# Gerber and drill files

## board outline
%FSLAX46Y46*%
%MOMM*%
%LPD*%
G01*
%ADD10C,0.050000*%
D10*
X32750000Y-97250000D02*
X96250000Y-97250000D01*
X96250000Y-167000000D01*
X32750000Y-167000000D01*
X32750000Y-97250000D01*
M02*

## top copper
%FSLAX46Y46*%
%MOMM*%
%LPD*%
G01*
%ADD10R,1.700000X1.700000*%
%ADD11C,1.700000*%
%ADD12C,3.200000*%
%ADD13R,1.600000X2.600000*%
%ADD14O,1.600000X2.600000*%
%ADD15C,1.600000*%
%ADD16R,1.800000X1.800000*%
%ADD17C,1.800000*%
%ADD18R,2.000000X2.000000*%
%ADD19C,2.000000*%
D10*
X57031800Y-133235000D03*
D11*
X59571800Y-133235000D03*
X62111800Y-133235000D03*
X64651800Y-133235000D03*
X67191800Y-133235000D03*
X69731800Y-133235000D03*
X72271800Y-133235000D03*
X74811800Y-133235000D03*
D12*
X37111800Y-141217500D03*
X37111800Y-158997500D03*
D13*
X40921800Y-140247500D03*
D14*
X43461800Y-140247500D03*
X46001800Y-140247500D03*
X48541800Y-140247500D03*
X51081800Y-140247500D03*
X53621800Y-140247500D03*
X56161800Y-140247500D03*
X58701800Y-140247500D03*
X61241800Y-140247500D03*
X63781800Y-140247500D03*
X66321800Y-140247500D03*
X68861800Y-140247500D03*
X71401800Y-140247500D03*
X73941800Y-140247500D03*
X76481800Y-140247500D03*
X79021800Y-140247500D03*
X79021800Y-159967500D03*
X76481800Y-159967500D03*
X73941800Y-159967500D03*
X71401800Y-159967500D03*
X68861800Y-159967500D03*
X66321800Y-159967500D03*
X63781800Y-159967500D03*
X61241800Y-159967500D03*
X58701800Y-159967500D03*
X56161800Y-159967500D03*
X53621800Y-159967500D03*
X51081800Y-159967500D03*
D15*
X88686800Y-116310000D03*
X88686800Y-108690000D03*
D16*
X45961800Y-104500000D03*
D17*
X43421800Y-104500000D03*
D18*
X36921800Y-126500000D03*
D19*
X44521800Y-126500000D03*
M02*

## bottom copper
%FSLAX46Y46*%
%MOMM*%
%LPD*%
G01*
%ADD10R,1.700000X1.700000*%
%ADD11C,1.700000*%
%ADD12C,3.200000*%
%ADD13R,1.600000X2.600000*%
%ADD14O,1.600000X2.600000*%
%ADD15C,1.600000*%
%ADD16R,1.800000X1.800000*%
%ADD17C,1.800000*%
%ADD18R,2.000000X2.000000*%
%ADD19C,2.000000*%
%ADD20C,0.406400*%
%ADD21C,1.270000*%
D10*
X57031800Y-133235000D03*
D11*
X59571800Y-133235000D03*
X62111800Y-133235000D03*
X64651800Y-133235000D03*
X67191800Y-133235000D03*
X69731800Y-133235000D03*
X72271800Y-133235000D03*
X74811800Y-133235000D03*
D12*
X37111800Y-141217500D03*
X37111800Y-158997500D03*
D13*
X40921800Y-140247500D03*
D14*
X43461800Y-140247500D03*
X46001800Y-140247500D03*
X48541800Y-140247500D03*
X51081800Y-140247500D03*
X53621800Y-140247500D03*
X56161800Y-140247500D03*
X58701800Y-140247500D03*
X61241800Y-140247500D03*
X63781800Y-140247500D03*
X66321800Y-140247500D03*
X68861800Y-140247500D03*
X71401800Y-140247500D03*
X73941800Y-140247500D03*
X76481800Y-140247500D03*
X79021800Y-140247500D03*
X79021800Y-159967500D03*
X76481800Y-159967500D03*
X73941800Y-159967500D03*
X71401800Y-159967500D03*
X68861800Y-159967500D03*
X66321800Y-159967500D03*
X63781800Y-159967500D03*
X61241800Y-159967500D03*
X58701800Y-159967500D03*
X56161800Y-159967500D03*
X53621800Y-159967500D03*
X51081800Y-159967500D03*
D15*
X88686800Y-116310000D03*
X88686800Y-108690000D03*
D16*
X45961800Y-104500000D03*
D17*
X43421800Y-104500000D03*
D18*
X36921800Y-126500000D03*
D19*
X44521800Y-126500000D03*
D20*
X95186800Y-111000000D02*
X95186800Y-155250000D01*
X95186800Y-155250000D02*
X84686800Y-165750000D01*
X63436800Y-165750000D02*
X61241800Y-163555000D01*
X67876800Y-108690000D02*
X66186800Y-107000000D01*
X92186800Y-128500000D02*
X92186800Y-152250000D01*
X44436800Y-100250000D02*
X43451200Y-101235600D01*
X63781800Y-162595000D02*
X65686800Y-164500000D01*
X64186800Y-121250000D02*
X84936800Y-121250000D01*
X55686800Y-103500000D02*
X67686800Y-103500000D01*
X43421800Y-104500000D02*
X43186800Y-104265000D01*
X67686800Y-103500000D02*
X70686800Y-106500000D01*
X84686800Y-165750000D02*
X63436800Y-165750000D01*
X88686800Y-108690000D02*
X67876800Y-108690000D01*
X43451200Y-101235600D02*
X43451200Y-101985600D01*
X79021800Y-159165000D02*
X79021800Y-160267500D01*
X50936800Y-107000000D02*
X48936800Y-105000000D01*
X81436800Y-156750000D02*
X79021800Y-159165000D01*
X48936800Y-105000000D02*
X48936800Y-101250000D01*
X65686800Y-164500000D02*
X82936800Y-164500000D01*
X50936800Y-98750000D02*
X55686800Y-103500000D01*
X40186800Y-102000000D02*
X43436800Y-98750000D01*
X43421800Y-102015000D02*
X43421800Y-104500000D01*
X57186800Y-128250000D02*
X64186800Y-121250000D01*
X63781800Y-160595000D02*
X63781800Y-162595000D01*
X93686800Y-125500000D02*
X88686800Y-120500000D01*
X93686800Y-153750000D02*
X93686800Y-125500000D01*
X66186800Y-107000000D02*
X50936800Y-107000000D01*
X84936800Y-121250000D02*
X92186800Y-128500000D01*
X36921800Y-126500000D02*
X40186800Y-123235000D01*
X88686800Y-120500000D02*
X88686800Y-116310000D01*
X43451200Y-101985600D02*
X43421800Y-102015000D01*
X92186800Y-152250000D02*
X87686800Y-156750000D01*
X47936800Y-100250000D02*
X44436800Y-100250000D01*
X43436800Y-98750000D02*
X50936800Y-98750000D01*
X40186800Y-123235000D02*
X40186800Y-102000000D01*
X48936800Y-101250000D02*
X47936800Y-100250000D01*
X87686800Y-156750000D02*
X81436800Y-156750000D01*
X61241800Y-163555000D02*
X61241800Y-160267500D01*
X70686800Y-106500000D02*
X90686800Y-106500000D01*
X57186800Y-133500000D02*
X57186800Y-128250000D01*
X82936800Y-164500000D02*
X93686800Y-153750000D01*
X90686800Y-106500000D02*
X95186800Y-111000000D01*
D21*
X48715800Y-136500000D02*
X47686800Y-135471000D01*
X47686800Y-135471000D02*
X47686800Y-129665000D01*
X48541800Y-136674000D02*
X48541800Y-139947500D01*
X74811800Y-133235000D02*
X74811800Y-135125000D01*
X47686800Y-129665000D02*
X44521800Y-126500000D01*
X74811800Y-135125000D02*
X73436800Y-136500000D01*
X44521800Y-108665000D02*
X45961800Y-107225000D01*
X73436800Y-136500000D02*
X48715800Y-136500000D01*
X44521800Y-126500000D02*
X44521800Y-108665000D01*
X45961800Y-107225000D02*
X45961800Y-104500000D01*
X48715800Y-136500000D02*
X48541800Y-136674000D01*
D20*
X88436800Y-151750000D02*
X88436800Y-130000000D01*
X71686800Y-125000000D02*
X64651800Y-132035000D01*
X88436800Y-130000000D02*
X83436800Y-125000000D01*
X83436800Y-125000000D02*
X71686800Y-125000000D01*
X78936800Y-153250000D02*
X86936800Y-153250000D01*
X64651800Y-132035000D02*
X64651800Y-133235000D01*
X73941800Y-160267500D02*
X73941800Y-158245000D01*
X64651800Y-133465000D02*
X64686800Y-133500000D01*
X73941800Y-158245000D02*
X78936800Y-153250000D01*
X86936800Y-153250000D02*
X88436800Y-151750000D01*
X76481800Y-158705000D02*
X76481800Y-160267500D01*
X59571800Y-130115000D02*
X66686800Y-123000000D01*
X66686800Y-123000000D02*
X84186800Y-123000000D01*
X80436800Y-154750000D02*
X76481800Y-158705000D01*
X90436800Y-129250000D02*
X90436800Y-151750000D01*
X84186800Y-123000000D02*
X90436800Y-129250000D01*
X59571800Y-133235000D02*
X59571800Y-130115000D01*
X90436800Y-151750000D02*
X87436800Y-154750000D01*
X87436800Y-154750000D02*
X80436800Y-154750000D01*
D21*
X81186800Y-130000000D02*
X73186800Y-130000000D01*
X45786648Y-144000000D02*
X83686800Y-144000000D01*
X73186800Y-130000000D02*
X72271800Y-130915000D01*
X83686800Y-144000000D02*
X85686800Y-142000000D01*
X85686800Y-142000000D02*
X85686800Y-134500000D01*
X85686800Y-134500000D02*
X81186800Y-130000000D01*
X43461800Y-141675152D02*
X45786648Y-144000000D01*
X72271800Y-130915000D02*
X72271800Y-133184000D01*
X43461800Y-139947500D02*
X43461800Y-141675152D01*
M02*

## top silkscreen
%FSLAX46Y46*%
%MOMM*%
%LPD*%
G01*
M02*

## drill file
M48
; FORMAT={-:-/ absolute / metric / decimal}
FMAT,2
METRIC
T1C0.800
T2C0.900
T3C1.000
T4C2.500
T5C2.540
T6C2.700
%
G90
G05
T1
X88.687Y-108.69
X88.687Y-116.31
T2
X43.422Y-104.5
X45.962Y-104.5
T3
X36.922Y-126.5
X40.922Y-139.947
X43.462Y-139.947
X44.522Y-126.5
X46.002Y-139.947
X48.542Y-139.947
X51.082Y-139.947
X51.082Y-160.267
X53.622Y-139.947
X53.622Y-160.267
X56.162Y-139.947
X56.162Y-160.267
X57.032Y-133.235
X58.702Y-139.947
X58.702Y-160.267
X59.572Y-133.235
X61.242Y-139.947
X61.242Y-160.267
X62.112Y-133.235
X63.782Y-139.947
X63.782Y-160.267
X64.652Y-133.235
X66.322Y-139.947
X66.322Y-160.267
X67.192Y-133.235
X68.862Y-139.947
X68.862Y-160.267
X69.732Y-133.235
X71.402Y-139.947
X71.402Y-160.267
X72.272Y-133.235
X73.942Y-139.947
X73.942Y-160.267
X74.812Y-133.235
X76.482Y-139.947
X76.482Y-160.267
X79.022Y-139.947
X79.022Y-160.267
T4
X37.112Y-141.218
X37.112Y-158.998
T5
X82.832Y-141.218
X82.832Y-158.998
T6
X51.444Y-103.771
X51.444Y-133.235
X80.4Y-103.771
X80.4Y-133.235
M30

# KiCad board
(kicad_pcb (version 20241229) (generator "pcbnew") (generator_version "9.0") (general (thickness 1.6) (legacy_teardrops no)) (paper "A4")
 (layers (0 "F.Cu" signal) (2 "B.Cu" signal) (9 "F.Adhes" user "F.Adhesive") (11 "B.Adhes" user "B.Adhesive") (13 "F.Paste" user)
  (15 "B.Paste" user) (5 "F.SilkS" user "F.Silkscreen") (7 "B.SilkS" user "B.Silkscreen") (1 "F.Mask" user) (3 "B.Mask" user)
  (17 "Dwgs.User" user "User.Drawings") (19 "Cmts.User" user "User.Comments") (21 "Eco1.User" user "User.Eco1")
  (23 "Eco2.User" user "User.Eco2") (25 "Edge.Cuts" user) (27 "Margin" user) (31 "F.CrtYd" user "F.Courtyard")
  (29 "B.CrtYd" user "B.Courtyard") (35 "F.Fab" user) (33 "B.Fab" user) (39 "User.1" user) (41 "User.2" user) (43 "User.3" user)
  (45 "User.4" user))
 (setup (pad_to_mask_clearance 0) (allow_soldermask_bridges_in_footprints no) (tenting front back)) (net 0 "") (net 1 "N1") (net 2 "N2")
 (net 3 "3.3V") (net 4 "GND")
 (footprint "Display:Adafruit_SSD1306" (layer "B.Cu") (at 57.0318 133.235)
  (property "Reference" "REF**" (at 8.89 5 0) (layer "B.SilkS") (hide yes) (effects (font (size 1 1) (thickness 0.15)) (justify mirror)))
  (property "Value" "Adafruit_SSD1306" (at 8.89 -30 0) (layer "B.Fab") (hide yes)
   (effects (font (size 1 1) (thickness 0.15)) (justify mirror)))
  (pad "" np_thru_hole circle (at -5.588 -29.464) (size 2.7 2.7) (drill 2.7) (layers "*.Cu" "*.Mask"))
  (pad "" np_thru_hole circle (at -5.588 0) (size 2.7 2.7) (drill 2.7) (layers "*.Cu" "*.Mask"))
  (pad "" np_thru_hole circle (at 23.368 -29.464) (size 2.7 2.7) (drill 2.7) (layers "*.Cu" "*.Mask"))
  (pad "" np_thru_hole circle (at 23.368 0) (size 2.7 2.7) (drill 2.7) (layers "*.Cu" "*.Mask"))
  (pad "1" thru_hole rect (at 0 0) (size 1.7 1.7) (drill 1) (layers "*.Cu" "*.Mask") (remove_unused_layers no))
  (pad "2" thru_hole circle (at 2.54 0) (size 1.7 1.7) (drill 1) (layers "*.Cu" "*.Mask") (remove_unused_layers no) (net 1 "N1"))
  (pad "3" thru_hole circle (at 5.08 0) (size 1.7 1.7) (drill 1) (layers "*.Cu" "*.Mask") (remove_unused_layers no))
  (pad "4" thru_hole circle (at 7.62 0) (size 1.7 1.7) (drill 1) (layers "*.Cu" "*.Mask") (remove_unused_layers no) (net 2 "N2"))
  (pad "5" thru_hole circle (at 10.16 0) (size 1.7 1.7) (drill 1) (layers "*.Cu" "*.Mask") (remove_unused_layers no))
  (pad "6" thru_hole circle (at 12.7 0) (size 1.7 1.7) (drill 1) (layers "*.Cu" "*.Mask") (remove_unused_layers no))
  (pad "7" thru_hole circle (at 15.24 0) (size 1.7 1.7) (drill 1) (layers "*.Cu" "*.Mask") (remove_unused_layers no) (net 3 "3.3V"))
  (pad "8" thru_hole circle (at 17.78 0) (size 1.7 1.7) (drill 1) (layers "*.Cu" "*.Mask") (remove_unused_layers no) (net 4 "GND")))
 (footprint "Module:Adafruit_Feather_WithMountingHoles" (layer "B.Cu") (at 40.9218 139.9475 -90)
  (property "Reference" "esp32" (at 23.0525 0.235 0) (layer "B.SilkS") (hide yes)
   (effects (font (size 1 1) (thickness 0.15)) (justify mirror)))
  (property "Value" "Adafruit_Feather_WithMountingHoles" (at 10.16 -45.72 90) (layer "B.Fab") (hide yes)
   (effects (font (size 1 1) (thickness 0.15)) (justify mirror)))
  (pad "" np_thru_hole circle (at 1.27 -41.91) (size 2.54 2.54) (drill 2.54) (layers "*.Cu" "*.Mask"))
  (pad "" np_thru_hole circle (at 1.27 3.81) (size 3.2 3.2) (drill 2.5) (layers "*.Cu" "*.Mask"))
  (pad "" np_thru_hole circle (at 19.05 -41.91) (size 2.54 2.54) (drill 2.54) (layers "*.Cu" "*.Mask"))
  (pad "" np_thru_hole circle (at 19.05 3.81) (size 3.2 3.2) (drill 2.5) (layers "*.Cu" "*.Mask"))
  (pad "1" thru_hole rect (at 0 0 270) (size 2.6 1.6) (drill 1 (offset 0.3 0)) (layers "*.Cu" "*.Mask") (remove_unused_layers no))
  (pad "2" thru_hole oval (at 0 -2.54 270) (size 2.6 1.6) (drill 1 (offset 0.3 0)) (layers "*.Cu" "*.Mask") (remove_unused_layers no)
   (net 3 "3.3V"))
  (pad "3" thru_hole oval (at 0 -5.08 270) (size 2.6 1.6) (drill 1 (offset 0.3 0)) (layers "*.Cu" "*.Mask") (remove_unused_layers no))
  (pad "4" thru_hole oval (at 0 -7.62 270) (size 2.6 1.6) (drill 1 (offset 0.3 0)) (layers "*.Cu" "*.Mask") (remove_unused_layers no)
   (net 4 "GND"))
  (pad "5" thru_hole oval (at 0 -10.16 270) (size 2.6 1.6) (drill 1 (offset 0.3 0)) (layers "*.Cu" "*.Mask") (remove_unused_layers no))
  (pad "6" thru_hole oval (at 0 -12.7 270) (size 2.6 1.6) (drill 1 (offset 0.3 0)) (layers "*.Cu" "*.Mask") (remove_unused_layers no))
  (pad "7" thru_hole oval (at 0 -15.24 270) (size 2.6 1.6) (drill 1 (offset 0.3 0)) (layers "*.Cu" "*.Mask") (remove_unused_layers no))
  (pad "8" thru_hole oval (at 0 -17.78 270) (size 2.6 1.6) (drill 1 (offset 0.3 0)) (layers "*.Cu" "*.Mask") (remove_unused_layers no))
  (pad "9" thru_hole oval (at 0 -20.32 270) (size 2.6 1.6) (drill 1 (offset 0.3 0)) (layers "*.Cu" "*.Mask") (remove_unused_layers no))
  (pad "10" thru_hole oval (at 0 -22.86 270) (size 2.6 1.6) (drill 1 (offset 0.3 0)) (layers "*.Cu" "*.Mask") (remove_unused_layers no))
  (pad "11" thru_hole oval (at 0 -25.4 270) (size 2.6 1.6) (drill 1 (offset 0.3 0)) (layers "*.Cu" "*.Mask") (remove_unused_layers no))
  (pad "12" thru_hole oval (at 0 -27.94 270) (size 2.6 1.6) (drill 1 (offset 0.3 0)) (layers "*.Cu" "*.Mask") (remove_unused_layers no))
  (pad "13" thru_hole oval (at 0 -30.48 270) (size 2.6 1.6) (drill 1 (offset 0.3 0)) (layers "*.Cu" "*.Mask") (remove_unused_layers no))
  (pad "14" thru_hole oval (at 0 -33.02 270) (size 2.6 1.6) (drill 1 (offset 0.3 0)) (layers "*.Cu" "*.Mask") (remove_unused_layers no))
  (pad "15" thru_hole oval (at 0 -35.56 270) (size 2.6 1.6) (drill 1 (offset 0.3 0)) (layers "*.Cu" "*.Mask") (remove_unused_layers no))
  (pad "16" thru_hole oval (at 0 -38.1 270) (size 2.6 1.6) (drill 1 (offset 0.3 0)) (layers "*.Cu" "*.Mask") (remove_unused_layers no))
  (pad "17" thru_hole oval (at 20.32 -38.1 90) (size 2.6 1.6) (drill 1 (offset 0.3 0)) (layers "*.Cu" "*.Mask") (remove_unused_layers no))
  (pad "18" thru_hole oval (at 20.32 -35.56 90) (size 2.6 1.6) (drill 1 (offset 0.3 0)) (layers "*.Cu" "*.Mask") (remove_unused_layers no)
   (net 1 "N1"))
  (pad "19" thru_hole oval (at 20.32 -33.02 90) (size 2.6 1.6) (drill 1 (offset 0.3 0)) (layers "*.Cu" "*.Mask") (remove_unused_layers no)
   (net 2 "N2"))
  (pad "20" thru_hole oval (at 20.32 -30.48 90) (size 2.6 1.6) (drill 1 (offset 0.3 0)) (layers "*.Cu" "*.Mask") (remove_unused_layers no))
  (pad "21" thru_hole oval (at 20.32 -27.94 90) (size 2.6 1.6) (drill 1 (offset 0.3 0)) (layers "*.Cu" "*.Mask") (remove_unused_layers no))
  (pad "22" thru_hole oval (at 20.32 -25.4 90) (size 2.6 1.6) (drill 1 (offset 0.3 0)) (layers "*.Cu" "*.Mask") (remove_unused_layers no))
  (pad "23" thru_hole oval (at 20.32 -22.86 90) (size 2.6 1.6) (drill 1 (offset 0.3 0)) (layers "*.Cu" "*.Mask") (remove_unused_layers no))
  (pad "24" thru_hole oval (at 20.32 -20.32 90) (size 2.6 1.6) (drill 1 (offset 0.3 0)) (layers "*.Cu" "*.Mask") (remove_unused_layers no))
  (pad "25" thru_hole oval (at 20.32 -17.78 90) (size 2.6 1.6) (drill 1 (offset 0.3 0)) (layers "*.Cu" "*.Mask") (remove_unused_layers no))
  (pad "26" thru_hole oval (at 20.32 -15.24 90) (size 2.6 1.6) (drill 1 (offset 0.3 0)) (layers "*.Cu" "*.Mask") (remove_unused_layers no))
  (pad "27" thru_hole oval (at 20.32 -12.7 90) (size 2.6 1.6) (drill 1 (offset 0.3 0)) (layers "*.Cu" "*.Mask") (remove_unused_layers no))
  (pad "28" thru_hole oval (at 20.32 -10.16 90) (size 2.6 1.6) (drill 1 (offset 0.3 0)) (layers "*.Cu" "*.Mask") (remove_unused_layers no)))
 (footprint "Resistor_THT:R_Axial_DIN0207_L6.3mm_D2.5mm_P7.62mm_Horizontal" (layer "B.Cu") (at 88.6868 116.31 90)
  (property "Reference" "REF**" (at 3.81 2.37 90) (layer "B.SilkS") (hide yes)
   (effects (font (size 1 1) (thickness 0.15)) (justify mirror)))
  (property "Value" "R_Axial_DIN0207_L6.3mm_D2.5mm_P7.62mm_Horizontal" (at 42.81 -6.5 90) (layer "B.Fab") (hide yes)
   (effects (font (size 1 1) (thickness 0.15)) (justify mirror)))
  (pad "1" thru_hole circle (at 0 0 90) (size 1.6 1.6) (drill 0.8) (layers "*.Cu" "*.Mask") (remove_unused_layers no))
  (pad "2" thru_hole circle (at 7.62 0 90) (size 1.6 1.6) (drill 0.8) (layers "*.Cu" "*.Mask") (remove_unused_layers no)))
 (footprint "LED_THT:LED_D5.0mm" (layer "B.Cu") (at 45.9618 104.5 180)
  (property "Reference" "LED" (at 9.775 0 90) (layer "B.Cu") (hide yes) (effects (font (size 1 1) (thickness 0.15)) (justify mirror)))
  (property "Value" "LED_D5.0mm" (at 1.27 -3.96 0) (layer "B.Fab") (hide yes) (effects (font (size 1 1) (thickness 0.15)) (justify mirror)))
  (pad "1" thru_hole rect (at 0 0 180) (size 1.8 1.8) (drill 0.9) (layers "*.Cu" "*.Mask") (remove_unused_layers no) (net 4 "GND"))
  (pad "2" thru_hole circle (at 2.54 0 180) (size 1.8 1.8) (drill 0.9) (layers "*.Cu" "*.Mask") (remove_unused_layers no)))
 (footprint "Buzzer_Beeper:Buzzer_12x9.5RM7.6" (layer "B.Cu") (at 36.9218 126.5)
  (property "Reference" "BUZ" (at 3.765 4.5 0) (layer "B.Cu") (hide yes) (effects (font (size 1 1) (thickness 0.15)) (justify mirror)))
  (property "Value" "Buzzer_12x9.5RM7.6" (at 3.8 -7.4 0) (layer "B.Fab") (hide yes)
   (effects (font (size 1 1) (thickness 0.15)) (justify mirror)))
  (pad "1" thru_hole rect (at 0 0) (size 2 2) (drill 1) (layers "*.Cu" "*.Mask") (remove_unused_layers no))
  (pad "2" thru_hole circle (at 7.6 0) (size 2 2) (drill 1) (layers "*.Cu" "*.Mask") (remove_unused_layers no) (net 4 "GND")))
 (gr_rect (start 32.75 97.25) (end 96.25 167) (stroke (width 0.05) (type default)) (fill no) (layer "Edge.Cuts"))
 (segment (start 95.1868 111) (end 95.1868 155.25) (width 0.4064) (layer "B.Cu") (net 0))
 (segment (start 95.1868 155.25) (end 84.6868 165.75) (width 0.4064) (layer "B.Cu") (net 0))
 (segment (start 63.4368 165.75) (end 61.2418 163.555) (width 0.4064) (layer "B.Cu") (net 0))
 (segment (start 67.8768 108.69) (end 66.1868 107) (width 0.4064) (layer "B.Cu") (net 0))
 (segment (start 92.1868 128.5) (end 92.1868 152.25) (width 0.4064) (layer "B.Cu") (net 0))
 (segment (start 44.4368 100.25) (end 43.4512 101.2356) (width 0.4064) (layer "B.Cu") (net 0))
 (segment (start 63.7818 162.595) (end 65.6868 164.5) (width 0.4064) (layer "B.Cu") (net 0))
 (segment (start 64.1868 121.25) (end 84.9368 121.25) (width 0.4064) (layer "B.Cu") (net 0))
 (segment (start 55.6868 103.5) (end 67.6868 103.5) (width 0.4064) (layer "B.Cu") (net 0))
 (segment (start 43.4218 104.5) (end 43.1868 104.265) (width 0.4064) (layer "B.Cu") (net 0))
 (segment (start 67.6868 103.5) (end 70.6868 106.5) (width 0.4064) (layer "B.Cu") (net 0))
 (segment (start 84.6868 165.75) (end 63.4368 165.75) (width 0.4064) (layer "B.Cu") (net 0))
 (segment (start 88.6868 108.69) (end 67.8768 108.69) (width 0.4064) (layer "B.Cu") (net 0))
 (segment (start 43.4512 101.2356) (end 43.4512 101.9856) (width 0.4064) (layer "B.Cu") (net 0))
 (segment (start 79.0218 159.165) (end 79.0218 160.2675) (width 0.4064) (layer "B.Cu") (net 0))
 (segment (start 50.9368 107) (end 48.9368 105) (width 0.4064) (layer "B.Cu") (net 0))
 (segment (start 81.4368 156.75) (end 79.0218 159.165) (width 0.4064) (layer "B.Cu") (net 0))
 (segment (start 48.9368 105) (end 48.9368 101.25) (width 0.4064) (layer "B.Cu") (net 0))
 (segment (start 65.6868 164.5) (end 82.9368 164.5) (width 0.4064) (layer "B.Cu") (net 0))
 (segment (start 50.9368 98.75) (end 55.6868 103.5) (width 0.4064) (layer "B.Cu") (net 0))
 (segment (start 40.1868 102) (end 43.4368 98.75) (width 0.4064) (layer "B.Cu") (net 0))
 (segment (start 43.4218 102.015) (end 43.4218 104.5) (width 0.4064) (layer "B.Cu") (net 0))
 (segment (start 57.1868 128.25) (end 64.1868 121.25) (width 0.4064) (layer "B.Cu") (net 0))
 (segment (start 63.7818 160.595) (end 63.7818 162.595) (width 0.4064) (layer "B.Cu") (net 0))
 (segment (start 93.6868 125.5) (end 88.6868 120.5) (width 0.4064) (layer "B.Cu") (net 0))
 (segment (start 93.6868 153.75) (end 93.6868 125.5) (width 0.4064) (layer "B.Cu") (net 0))
 (segment (start 66.1868 107) (end 50.9368 107) (width 0.4064) (layer "B.Cu") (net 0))
 (segment (start 84.9368 121.25) (end 92.1868 128.5) (width 0.4064) (layer "B.Cu") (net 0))
 (segment (start 36.9218 126.5) (end 40.1868 123.235) (width 0.4064) (layer "B.Cu") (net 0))
 (segment (start 88.6868 120.5) (end 88.6868 116.31) (width 0.4064) (layer "B.Cu") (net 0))
 (segment (start 43.4512 101.9856) (end 43.4218 102.015) (width 0.4064) (layer "B.Cu") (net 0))
 (segment (start 92.1868 152.25) (end 87.6868 156.75) (width 0.4064) (layer "B.Cu") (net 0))
 (segment (start 47.9368 100.25) (end 44.4368 100.25) (width 0.4064) (layer "B.Cu") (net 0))
 (segment (start 43.4368 98.75) (end 50.9368 98.75) (width 0.4064) (layer "B.Cu") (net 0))
 (segment (start 40.1868 123.235) (end 40.1868 102) (width 0.4064) (layer "B.Cu") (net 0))
 (segment (start 48.9368 101.25) (end 47.9368 100.25) (width 0.4064) (layer "B.Cu") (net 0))
 (segment (start 87.6868 156.75) (end 81.4368 156.75) (width 0.4064) (layer "B.Cu") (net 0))
 (segment (start 61.2418 163.555) (end 61.2418 160.2675) (width 0.4064) (layer "B.Cu") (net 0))
 (segment (start 70.6868 106.5) (end 90.6868 106.5) (width 0.4064) (layer "B.Cu") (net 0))
 (segment (start 57.1868 133.5) (end 57.1868 128.25) (width 0.4064) (layer "B.Cu") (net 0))
 (segment (start 82.9368 164.5) (end 93.6868 153.75) (width 0.4064) (layer "B.Cu") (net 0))
 (segment (start 90.6868 106.5) (end 95.1868 111) (width 0.4064) (layer "B.Cu") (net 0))
 (segment (start 48.7158 136.5) (end 47.6868 135.471) (width 1.27) (layer "B.Cu") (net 4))
 (segment (start 47.6868 135.471) (end 47.6868 129.665) (width 1.27) (layer "B.Cu") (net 4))
 (segment (start 48.5418 136.674) (end 48.5418 139.9475) (width 1.27) (layer "B.Cu") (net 4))
 (segment (start 74.8118 133.235) (end 74.8118 135.125) (width 1.27) (layer "B.Cu") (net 4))
 (segment (start 47.6868 129.665) (end 44.5218 126.5) (width 1.27) (layer "B.Cu") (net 4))
 (segment (start 74.8118 135.125) (end 73.4368 136.5) (width 1.27) (layer "B.Cu") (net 4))
 (segment (start 44.5218 108.665) (end 45.9618 107.225) (width 1.27) (layer "B.Cu") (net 4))
 (segment (start 73.4368 136.5) (end 48.7158 136.5) (width 1.27) (layer "B.Cu") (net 4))
 (segment (start 44.5218 126.5) (end 44.5218 108.665) (width 1.27) (layer "B.Cu") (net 4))
 (segment (start 45.9618 107.225) (end 45.9618 104.5) (width 1.27) (layer "B.Cu") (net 4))
 (segment (start 48.7158 136.5) (end 48.5418 136.674) (width 1.27) (layer "B.Cu") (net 4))
 (segment (start 88.4368 151.75) (end 88.4368 130) (width 0.4064) (layer "B.Cu") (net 2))
 (segment (start 71.6868 125) (end 64.6518 132.035) (width 0.4064) (layer "B.Cu") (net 2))
 (segment (start 88.4368 130) (end 83.4368 125) (width 0.4064) (layer "B.Cu") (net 2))
 (segment (start 83.4368 125) (end 71.6868 125) (width 0.4064) (layer "B.Cu") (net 2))
 (segment (start 78.9368 153.25) (end 86.9368 153.25) (width 0.4064) (layer "B.Cu") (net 2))
 (segment (start 64.6518 132.035) (end 64.6518 133.235) (width 0.4064) (layer "B.Cu") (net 2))
 (segment (start 73.9418 160.2675) (end 73.9418 158.245) (width 0.4064) (layer "B.Cu") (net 2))
 (segment (start 64.6518 133.465) (end 64.6868 133.5) (width 0.4064) (layer "B.Cu") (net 2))
 (segment (start 73.9418 158.245) (end 78.9368 153.25) (width 0.4064) (layer "B.Cu") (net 2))
 (segment (start 86.9368 153.25) (end 88.4368 151.75) (width 0.4064) (layer "B.Cu") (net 2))
 (segment (start 76.4818 158.705) (end 76.4818 160.2675) (width 0.4064) (layer "B.Cu") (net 1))
 (segment (start 59.5718 130.115) (end 66.6868 123) (width 0.4064) (layer "B.Cu") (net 1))
 (segment (start 66.6868 123) (end 84.1868 123) (width 0.4064) (layer "B.Cu") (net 1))
 (segment (start 80.4368 154.75) (end 76.4818 158.705) (width 0.4064) (layer "B.Cu") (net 1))
 (segment (start 90.4368 129.25) (end 90.4368 151.75) (width 0.4064) (layer "B.Cu") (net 1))
 (segment (start 84.1868 123) (end 90.4368 129.25) (width 0.4064) (layer "B.Cu") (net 1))
 (segment (start 59.5718 133.235) (end 59.5718 130.115) (width 0.4064) (layer "B.Cu") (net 1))
 (segment (start 90.4368 151.75) (end 87.4368 154.75) (width 0.4064) (layer "B.Cu") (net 1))
 (segment (start 87.4368 154.75) (end 80.4368 154.75) (width 0.4064) (layer "B.Cu") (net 1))
 (segment (start 81.1868 130) (end 73.1868 130) (width 1.27) (layer "B.Cu") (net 3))
 (segment (start 45.786648 144) (end 83.6868 144) (width 1.27) (layer "B.Cu") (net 3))
 (segment (start 73.1868 130) (end 72.2718 130.915) (width 1.27) (layer "B.Cu") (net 3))
 (segment (start 83.6868 144) (end 85.6868 142) (width 1.27) (layer "B.Cu") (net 3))
 (segment (start 85.6868 142) (end 85.6868 134.5) (width 1.27) (layer "B.Cu") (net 3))
 (segment (start 85.6868 134.5) (end 81.1868 130) (width 1.27) (layer "B.Cu") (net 3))
 (segment (start 43.4618 141.675152) (end 45.786648 144) (width 1.27) (layer "B.Cu") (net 3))
 (segment (start 72.2718 130.915) (end 72.2718 133.184) (width 1.27) (layer "B.Cu") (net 3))
 (segment (start 43.4618 139.9475) (end 43.4618 141.675152) (width 1.27) (layer "B.Cu") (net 3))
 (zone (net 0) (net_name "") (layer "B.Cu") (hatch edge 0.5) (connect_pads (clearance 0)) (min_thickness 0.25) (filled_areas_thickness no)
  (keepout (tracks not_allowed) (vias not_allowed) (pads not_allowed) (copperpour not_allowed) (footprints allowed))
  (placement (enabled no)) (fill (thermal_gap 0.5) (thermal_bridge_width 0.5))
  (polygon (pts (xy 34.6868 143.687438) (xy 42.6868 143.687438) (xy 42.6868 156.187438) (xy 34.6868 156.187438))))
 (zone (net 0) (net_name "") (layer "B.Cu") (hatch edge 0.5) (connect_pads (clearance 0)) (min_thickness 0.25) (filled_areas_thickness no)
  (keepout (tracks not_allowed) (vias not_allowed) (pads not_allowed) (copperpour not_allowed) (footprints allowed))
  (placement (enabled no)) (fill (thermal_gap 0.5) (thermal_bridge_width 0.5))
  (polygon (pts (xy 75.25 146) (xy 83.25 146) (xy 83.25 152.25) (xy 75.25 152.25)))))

